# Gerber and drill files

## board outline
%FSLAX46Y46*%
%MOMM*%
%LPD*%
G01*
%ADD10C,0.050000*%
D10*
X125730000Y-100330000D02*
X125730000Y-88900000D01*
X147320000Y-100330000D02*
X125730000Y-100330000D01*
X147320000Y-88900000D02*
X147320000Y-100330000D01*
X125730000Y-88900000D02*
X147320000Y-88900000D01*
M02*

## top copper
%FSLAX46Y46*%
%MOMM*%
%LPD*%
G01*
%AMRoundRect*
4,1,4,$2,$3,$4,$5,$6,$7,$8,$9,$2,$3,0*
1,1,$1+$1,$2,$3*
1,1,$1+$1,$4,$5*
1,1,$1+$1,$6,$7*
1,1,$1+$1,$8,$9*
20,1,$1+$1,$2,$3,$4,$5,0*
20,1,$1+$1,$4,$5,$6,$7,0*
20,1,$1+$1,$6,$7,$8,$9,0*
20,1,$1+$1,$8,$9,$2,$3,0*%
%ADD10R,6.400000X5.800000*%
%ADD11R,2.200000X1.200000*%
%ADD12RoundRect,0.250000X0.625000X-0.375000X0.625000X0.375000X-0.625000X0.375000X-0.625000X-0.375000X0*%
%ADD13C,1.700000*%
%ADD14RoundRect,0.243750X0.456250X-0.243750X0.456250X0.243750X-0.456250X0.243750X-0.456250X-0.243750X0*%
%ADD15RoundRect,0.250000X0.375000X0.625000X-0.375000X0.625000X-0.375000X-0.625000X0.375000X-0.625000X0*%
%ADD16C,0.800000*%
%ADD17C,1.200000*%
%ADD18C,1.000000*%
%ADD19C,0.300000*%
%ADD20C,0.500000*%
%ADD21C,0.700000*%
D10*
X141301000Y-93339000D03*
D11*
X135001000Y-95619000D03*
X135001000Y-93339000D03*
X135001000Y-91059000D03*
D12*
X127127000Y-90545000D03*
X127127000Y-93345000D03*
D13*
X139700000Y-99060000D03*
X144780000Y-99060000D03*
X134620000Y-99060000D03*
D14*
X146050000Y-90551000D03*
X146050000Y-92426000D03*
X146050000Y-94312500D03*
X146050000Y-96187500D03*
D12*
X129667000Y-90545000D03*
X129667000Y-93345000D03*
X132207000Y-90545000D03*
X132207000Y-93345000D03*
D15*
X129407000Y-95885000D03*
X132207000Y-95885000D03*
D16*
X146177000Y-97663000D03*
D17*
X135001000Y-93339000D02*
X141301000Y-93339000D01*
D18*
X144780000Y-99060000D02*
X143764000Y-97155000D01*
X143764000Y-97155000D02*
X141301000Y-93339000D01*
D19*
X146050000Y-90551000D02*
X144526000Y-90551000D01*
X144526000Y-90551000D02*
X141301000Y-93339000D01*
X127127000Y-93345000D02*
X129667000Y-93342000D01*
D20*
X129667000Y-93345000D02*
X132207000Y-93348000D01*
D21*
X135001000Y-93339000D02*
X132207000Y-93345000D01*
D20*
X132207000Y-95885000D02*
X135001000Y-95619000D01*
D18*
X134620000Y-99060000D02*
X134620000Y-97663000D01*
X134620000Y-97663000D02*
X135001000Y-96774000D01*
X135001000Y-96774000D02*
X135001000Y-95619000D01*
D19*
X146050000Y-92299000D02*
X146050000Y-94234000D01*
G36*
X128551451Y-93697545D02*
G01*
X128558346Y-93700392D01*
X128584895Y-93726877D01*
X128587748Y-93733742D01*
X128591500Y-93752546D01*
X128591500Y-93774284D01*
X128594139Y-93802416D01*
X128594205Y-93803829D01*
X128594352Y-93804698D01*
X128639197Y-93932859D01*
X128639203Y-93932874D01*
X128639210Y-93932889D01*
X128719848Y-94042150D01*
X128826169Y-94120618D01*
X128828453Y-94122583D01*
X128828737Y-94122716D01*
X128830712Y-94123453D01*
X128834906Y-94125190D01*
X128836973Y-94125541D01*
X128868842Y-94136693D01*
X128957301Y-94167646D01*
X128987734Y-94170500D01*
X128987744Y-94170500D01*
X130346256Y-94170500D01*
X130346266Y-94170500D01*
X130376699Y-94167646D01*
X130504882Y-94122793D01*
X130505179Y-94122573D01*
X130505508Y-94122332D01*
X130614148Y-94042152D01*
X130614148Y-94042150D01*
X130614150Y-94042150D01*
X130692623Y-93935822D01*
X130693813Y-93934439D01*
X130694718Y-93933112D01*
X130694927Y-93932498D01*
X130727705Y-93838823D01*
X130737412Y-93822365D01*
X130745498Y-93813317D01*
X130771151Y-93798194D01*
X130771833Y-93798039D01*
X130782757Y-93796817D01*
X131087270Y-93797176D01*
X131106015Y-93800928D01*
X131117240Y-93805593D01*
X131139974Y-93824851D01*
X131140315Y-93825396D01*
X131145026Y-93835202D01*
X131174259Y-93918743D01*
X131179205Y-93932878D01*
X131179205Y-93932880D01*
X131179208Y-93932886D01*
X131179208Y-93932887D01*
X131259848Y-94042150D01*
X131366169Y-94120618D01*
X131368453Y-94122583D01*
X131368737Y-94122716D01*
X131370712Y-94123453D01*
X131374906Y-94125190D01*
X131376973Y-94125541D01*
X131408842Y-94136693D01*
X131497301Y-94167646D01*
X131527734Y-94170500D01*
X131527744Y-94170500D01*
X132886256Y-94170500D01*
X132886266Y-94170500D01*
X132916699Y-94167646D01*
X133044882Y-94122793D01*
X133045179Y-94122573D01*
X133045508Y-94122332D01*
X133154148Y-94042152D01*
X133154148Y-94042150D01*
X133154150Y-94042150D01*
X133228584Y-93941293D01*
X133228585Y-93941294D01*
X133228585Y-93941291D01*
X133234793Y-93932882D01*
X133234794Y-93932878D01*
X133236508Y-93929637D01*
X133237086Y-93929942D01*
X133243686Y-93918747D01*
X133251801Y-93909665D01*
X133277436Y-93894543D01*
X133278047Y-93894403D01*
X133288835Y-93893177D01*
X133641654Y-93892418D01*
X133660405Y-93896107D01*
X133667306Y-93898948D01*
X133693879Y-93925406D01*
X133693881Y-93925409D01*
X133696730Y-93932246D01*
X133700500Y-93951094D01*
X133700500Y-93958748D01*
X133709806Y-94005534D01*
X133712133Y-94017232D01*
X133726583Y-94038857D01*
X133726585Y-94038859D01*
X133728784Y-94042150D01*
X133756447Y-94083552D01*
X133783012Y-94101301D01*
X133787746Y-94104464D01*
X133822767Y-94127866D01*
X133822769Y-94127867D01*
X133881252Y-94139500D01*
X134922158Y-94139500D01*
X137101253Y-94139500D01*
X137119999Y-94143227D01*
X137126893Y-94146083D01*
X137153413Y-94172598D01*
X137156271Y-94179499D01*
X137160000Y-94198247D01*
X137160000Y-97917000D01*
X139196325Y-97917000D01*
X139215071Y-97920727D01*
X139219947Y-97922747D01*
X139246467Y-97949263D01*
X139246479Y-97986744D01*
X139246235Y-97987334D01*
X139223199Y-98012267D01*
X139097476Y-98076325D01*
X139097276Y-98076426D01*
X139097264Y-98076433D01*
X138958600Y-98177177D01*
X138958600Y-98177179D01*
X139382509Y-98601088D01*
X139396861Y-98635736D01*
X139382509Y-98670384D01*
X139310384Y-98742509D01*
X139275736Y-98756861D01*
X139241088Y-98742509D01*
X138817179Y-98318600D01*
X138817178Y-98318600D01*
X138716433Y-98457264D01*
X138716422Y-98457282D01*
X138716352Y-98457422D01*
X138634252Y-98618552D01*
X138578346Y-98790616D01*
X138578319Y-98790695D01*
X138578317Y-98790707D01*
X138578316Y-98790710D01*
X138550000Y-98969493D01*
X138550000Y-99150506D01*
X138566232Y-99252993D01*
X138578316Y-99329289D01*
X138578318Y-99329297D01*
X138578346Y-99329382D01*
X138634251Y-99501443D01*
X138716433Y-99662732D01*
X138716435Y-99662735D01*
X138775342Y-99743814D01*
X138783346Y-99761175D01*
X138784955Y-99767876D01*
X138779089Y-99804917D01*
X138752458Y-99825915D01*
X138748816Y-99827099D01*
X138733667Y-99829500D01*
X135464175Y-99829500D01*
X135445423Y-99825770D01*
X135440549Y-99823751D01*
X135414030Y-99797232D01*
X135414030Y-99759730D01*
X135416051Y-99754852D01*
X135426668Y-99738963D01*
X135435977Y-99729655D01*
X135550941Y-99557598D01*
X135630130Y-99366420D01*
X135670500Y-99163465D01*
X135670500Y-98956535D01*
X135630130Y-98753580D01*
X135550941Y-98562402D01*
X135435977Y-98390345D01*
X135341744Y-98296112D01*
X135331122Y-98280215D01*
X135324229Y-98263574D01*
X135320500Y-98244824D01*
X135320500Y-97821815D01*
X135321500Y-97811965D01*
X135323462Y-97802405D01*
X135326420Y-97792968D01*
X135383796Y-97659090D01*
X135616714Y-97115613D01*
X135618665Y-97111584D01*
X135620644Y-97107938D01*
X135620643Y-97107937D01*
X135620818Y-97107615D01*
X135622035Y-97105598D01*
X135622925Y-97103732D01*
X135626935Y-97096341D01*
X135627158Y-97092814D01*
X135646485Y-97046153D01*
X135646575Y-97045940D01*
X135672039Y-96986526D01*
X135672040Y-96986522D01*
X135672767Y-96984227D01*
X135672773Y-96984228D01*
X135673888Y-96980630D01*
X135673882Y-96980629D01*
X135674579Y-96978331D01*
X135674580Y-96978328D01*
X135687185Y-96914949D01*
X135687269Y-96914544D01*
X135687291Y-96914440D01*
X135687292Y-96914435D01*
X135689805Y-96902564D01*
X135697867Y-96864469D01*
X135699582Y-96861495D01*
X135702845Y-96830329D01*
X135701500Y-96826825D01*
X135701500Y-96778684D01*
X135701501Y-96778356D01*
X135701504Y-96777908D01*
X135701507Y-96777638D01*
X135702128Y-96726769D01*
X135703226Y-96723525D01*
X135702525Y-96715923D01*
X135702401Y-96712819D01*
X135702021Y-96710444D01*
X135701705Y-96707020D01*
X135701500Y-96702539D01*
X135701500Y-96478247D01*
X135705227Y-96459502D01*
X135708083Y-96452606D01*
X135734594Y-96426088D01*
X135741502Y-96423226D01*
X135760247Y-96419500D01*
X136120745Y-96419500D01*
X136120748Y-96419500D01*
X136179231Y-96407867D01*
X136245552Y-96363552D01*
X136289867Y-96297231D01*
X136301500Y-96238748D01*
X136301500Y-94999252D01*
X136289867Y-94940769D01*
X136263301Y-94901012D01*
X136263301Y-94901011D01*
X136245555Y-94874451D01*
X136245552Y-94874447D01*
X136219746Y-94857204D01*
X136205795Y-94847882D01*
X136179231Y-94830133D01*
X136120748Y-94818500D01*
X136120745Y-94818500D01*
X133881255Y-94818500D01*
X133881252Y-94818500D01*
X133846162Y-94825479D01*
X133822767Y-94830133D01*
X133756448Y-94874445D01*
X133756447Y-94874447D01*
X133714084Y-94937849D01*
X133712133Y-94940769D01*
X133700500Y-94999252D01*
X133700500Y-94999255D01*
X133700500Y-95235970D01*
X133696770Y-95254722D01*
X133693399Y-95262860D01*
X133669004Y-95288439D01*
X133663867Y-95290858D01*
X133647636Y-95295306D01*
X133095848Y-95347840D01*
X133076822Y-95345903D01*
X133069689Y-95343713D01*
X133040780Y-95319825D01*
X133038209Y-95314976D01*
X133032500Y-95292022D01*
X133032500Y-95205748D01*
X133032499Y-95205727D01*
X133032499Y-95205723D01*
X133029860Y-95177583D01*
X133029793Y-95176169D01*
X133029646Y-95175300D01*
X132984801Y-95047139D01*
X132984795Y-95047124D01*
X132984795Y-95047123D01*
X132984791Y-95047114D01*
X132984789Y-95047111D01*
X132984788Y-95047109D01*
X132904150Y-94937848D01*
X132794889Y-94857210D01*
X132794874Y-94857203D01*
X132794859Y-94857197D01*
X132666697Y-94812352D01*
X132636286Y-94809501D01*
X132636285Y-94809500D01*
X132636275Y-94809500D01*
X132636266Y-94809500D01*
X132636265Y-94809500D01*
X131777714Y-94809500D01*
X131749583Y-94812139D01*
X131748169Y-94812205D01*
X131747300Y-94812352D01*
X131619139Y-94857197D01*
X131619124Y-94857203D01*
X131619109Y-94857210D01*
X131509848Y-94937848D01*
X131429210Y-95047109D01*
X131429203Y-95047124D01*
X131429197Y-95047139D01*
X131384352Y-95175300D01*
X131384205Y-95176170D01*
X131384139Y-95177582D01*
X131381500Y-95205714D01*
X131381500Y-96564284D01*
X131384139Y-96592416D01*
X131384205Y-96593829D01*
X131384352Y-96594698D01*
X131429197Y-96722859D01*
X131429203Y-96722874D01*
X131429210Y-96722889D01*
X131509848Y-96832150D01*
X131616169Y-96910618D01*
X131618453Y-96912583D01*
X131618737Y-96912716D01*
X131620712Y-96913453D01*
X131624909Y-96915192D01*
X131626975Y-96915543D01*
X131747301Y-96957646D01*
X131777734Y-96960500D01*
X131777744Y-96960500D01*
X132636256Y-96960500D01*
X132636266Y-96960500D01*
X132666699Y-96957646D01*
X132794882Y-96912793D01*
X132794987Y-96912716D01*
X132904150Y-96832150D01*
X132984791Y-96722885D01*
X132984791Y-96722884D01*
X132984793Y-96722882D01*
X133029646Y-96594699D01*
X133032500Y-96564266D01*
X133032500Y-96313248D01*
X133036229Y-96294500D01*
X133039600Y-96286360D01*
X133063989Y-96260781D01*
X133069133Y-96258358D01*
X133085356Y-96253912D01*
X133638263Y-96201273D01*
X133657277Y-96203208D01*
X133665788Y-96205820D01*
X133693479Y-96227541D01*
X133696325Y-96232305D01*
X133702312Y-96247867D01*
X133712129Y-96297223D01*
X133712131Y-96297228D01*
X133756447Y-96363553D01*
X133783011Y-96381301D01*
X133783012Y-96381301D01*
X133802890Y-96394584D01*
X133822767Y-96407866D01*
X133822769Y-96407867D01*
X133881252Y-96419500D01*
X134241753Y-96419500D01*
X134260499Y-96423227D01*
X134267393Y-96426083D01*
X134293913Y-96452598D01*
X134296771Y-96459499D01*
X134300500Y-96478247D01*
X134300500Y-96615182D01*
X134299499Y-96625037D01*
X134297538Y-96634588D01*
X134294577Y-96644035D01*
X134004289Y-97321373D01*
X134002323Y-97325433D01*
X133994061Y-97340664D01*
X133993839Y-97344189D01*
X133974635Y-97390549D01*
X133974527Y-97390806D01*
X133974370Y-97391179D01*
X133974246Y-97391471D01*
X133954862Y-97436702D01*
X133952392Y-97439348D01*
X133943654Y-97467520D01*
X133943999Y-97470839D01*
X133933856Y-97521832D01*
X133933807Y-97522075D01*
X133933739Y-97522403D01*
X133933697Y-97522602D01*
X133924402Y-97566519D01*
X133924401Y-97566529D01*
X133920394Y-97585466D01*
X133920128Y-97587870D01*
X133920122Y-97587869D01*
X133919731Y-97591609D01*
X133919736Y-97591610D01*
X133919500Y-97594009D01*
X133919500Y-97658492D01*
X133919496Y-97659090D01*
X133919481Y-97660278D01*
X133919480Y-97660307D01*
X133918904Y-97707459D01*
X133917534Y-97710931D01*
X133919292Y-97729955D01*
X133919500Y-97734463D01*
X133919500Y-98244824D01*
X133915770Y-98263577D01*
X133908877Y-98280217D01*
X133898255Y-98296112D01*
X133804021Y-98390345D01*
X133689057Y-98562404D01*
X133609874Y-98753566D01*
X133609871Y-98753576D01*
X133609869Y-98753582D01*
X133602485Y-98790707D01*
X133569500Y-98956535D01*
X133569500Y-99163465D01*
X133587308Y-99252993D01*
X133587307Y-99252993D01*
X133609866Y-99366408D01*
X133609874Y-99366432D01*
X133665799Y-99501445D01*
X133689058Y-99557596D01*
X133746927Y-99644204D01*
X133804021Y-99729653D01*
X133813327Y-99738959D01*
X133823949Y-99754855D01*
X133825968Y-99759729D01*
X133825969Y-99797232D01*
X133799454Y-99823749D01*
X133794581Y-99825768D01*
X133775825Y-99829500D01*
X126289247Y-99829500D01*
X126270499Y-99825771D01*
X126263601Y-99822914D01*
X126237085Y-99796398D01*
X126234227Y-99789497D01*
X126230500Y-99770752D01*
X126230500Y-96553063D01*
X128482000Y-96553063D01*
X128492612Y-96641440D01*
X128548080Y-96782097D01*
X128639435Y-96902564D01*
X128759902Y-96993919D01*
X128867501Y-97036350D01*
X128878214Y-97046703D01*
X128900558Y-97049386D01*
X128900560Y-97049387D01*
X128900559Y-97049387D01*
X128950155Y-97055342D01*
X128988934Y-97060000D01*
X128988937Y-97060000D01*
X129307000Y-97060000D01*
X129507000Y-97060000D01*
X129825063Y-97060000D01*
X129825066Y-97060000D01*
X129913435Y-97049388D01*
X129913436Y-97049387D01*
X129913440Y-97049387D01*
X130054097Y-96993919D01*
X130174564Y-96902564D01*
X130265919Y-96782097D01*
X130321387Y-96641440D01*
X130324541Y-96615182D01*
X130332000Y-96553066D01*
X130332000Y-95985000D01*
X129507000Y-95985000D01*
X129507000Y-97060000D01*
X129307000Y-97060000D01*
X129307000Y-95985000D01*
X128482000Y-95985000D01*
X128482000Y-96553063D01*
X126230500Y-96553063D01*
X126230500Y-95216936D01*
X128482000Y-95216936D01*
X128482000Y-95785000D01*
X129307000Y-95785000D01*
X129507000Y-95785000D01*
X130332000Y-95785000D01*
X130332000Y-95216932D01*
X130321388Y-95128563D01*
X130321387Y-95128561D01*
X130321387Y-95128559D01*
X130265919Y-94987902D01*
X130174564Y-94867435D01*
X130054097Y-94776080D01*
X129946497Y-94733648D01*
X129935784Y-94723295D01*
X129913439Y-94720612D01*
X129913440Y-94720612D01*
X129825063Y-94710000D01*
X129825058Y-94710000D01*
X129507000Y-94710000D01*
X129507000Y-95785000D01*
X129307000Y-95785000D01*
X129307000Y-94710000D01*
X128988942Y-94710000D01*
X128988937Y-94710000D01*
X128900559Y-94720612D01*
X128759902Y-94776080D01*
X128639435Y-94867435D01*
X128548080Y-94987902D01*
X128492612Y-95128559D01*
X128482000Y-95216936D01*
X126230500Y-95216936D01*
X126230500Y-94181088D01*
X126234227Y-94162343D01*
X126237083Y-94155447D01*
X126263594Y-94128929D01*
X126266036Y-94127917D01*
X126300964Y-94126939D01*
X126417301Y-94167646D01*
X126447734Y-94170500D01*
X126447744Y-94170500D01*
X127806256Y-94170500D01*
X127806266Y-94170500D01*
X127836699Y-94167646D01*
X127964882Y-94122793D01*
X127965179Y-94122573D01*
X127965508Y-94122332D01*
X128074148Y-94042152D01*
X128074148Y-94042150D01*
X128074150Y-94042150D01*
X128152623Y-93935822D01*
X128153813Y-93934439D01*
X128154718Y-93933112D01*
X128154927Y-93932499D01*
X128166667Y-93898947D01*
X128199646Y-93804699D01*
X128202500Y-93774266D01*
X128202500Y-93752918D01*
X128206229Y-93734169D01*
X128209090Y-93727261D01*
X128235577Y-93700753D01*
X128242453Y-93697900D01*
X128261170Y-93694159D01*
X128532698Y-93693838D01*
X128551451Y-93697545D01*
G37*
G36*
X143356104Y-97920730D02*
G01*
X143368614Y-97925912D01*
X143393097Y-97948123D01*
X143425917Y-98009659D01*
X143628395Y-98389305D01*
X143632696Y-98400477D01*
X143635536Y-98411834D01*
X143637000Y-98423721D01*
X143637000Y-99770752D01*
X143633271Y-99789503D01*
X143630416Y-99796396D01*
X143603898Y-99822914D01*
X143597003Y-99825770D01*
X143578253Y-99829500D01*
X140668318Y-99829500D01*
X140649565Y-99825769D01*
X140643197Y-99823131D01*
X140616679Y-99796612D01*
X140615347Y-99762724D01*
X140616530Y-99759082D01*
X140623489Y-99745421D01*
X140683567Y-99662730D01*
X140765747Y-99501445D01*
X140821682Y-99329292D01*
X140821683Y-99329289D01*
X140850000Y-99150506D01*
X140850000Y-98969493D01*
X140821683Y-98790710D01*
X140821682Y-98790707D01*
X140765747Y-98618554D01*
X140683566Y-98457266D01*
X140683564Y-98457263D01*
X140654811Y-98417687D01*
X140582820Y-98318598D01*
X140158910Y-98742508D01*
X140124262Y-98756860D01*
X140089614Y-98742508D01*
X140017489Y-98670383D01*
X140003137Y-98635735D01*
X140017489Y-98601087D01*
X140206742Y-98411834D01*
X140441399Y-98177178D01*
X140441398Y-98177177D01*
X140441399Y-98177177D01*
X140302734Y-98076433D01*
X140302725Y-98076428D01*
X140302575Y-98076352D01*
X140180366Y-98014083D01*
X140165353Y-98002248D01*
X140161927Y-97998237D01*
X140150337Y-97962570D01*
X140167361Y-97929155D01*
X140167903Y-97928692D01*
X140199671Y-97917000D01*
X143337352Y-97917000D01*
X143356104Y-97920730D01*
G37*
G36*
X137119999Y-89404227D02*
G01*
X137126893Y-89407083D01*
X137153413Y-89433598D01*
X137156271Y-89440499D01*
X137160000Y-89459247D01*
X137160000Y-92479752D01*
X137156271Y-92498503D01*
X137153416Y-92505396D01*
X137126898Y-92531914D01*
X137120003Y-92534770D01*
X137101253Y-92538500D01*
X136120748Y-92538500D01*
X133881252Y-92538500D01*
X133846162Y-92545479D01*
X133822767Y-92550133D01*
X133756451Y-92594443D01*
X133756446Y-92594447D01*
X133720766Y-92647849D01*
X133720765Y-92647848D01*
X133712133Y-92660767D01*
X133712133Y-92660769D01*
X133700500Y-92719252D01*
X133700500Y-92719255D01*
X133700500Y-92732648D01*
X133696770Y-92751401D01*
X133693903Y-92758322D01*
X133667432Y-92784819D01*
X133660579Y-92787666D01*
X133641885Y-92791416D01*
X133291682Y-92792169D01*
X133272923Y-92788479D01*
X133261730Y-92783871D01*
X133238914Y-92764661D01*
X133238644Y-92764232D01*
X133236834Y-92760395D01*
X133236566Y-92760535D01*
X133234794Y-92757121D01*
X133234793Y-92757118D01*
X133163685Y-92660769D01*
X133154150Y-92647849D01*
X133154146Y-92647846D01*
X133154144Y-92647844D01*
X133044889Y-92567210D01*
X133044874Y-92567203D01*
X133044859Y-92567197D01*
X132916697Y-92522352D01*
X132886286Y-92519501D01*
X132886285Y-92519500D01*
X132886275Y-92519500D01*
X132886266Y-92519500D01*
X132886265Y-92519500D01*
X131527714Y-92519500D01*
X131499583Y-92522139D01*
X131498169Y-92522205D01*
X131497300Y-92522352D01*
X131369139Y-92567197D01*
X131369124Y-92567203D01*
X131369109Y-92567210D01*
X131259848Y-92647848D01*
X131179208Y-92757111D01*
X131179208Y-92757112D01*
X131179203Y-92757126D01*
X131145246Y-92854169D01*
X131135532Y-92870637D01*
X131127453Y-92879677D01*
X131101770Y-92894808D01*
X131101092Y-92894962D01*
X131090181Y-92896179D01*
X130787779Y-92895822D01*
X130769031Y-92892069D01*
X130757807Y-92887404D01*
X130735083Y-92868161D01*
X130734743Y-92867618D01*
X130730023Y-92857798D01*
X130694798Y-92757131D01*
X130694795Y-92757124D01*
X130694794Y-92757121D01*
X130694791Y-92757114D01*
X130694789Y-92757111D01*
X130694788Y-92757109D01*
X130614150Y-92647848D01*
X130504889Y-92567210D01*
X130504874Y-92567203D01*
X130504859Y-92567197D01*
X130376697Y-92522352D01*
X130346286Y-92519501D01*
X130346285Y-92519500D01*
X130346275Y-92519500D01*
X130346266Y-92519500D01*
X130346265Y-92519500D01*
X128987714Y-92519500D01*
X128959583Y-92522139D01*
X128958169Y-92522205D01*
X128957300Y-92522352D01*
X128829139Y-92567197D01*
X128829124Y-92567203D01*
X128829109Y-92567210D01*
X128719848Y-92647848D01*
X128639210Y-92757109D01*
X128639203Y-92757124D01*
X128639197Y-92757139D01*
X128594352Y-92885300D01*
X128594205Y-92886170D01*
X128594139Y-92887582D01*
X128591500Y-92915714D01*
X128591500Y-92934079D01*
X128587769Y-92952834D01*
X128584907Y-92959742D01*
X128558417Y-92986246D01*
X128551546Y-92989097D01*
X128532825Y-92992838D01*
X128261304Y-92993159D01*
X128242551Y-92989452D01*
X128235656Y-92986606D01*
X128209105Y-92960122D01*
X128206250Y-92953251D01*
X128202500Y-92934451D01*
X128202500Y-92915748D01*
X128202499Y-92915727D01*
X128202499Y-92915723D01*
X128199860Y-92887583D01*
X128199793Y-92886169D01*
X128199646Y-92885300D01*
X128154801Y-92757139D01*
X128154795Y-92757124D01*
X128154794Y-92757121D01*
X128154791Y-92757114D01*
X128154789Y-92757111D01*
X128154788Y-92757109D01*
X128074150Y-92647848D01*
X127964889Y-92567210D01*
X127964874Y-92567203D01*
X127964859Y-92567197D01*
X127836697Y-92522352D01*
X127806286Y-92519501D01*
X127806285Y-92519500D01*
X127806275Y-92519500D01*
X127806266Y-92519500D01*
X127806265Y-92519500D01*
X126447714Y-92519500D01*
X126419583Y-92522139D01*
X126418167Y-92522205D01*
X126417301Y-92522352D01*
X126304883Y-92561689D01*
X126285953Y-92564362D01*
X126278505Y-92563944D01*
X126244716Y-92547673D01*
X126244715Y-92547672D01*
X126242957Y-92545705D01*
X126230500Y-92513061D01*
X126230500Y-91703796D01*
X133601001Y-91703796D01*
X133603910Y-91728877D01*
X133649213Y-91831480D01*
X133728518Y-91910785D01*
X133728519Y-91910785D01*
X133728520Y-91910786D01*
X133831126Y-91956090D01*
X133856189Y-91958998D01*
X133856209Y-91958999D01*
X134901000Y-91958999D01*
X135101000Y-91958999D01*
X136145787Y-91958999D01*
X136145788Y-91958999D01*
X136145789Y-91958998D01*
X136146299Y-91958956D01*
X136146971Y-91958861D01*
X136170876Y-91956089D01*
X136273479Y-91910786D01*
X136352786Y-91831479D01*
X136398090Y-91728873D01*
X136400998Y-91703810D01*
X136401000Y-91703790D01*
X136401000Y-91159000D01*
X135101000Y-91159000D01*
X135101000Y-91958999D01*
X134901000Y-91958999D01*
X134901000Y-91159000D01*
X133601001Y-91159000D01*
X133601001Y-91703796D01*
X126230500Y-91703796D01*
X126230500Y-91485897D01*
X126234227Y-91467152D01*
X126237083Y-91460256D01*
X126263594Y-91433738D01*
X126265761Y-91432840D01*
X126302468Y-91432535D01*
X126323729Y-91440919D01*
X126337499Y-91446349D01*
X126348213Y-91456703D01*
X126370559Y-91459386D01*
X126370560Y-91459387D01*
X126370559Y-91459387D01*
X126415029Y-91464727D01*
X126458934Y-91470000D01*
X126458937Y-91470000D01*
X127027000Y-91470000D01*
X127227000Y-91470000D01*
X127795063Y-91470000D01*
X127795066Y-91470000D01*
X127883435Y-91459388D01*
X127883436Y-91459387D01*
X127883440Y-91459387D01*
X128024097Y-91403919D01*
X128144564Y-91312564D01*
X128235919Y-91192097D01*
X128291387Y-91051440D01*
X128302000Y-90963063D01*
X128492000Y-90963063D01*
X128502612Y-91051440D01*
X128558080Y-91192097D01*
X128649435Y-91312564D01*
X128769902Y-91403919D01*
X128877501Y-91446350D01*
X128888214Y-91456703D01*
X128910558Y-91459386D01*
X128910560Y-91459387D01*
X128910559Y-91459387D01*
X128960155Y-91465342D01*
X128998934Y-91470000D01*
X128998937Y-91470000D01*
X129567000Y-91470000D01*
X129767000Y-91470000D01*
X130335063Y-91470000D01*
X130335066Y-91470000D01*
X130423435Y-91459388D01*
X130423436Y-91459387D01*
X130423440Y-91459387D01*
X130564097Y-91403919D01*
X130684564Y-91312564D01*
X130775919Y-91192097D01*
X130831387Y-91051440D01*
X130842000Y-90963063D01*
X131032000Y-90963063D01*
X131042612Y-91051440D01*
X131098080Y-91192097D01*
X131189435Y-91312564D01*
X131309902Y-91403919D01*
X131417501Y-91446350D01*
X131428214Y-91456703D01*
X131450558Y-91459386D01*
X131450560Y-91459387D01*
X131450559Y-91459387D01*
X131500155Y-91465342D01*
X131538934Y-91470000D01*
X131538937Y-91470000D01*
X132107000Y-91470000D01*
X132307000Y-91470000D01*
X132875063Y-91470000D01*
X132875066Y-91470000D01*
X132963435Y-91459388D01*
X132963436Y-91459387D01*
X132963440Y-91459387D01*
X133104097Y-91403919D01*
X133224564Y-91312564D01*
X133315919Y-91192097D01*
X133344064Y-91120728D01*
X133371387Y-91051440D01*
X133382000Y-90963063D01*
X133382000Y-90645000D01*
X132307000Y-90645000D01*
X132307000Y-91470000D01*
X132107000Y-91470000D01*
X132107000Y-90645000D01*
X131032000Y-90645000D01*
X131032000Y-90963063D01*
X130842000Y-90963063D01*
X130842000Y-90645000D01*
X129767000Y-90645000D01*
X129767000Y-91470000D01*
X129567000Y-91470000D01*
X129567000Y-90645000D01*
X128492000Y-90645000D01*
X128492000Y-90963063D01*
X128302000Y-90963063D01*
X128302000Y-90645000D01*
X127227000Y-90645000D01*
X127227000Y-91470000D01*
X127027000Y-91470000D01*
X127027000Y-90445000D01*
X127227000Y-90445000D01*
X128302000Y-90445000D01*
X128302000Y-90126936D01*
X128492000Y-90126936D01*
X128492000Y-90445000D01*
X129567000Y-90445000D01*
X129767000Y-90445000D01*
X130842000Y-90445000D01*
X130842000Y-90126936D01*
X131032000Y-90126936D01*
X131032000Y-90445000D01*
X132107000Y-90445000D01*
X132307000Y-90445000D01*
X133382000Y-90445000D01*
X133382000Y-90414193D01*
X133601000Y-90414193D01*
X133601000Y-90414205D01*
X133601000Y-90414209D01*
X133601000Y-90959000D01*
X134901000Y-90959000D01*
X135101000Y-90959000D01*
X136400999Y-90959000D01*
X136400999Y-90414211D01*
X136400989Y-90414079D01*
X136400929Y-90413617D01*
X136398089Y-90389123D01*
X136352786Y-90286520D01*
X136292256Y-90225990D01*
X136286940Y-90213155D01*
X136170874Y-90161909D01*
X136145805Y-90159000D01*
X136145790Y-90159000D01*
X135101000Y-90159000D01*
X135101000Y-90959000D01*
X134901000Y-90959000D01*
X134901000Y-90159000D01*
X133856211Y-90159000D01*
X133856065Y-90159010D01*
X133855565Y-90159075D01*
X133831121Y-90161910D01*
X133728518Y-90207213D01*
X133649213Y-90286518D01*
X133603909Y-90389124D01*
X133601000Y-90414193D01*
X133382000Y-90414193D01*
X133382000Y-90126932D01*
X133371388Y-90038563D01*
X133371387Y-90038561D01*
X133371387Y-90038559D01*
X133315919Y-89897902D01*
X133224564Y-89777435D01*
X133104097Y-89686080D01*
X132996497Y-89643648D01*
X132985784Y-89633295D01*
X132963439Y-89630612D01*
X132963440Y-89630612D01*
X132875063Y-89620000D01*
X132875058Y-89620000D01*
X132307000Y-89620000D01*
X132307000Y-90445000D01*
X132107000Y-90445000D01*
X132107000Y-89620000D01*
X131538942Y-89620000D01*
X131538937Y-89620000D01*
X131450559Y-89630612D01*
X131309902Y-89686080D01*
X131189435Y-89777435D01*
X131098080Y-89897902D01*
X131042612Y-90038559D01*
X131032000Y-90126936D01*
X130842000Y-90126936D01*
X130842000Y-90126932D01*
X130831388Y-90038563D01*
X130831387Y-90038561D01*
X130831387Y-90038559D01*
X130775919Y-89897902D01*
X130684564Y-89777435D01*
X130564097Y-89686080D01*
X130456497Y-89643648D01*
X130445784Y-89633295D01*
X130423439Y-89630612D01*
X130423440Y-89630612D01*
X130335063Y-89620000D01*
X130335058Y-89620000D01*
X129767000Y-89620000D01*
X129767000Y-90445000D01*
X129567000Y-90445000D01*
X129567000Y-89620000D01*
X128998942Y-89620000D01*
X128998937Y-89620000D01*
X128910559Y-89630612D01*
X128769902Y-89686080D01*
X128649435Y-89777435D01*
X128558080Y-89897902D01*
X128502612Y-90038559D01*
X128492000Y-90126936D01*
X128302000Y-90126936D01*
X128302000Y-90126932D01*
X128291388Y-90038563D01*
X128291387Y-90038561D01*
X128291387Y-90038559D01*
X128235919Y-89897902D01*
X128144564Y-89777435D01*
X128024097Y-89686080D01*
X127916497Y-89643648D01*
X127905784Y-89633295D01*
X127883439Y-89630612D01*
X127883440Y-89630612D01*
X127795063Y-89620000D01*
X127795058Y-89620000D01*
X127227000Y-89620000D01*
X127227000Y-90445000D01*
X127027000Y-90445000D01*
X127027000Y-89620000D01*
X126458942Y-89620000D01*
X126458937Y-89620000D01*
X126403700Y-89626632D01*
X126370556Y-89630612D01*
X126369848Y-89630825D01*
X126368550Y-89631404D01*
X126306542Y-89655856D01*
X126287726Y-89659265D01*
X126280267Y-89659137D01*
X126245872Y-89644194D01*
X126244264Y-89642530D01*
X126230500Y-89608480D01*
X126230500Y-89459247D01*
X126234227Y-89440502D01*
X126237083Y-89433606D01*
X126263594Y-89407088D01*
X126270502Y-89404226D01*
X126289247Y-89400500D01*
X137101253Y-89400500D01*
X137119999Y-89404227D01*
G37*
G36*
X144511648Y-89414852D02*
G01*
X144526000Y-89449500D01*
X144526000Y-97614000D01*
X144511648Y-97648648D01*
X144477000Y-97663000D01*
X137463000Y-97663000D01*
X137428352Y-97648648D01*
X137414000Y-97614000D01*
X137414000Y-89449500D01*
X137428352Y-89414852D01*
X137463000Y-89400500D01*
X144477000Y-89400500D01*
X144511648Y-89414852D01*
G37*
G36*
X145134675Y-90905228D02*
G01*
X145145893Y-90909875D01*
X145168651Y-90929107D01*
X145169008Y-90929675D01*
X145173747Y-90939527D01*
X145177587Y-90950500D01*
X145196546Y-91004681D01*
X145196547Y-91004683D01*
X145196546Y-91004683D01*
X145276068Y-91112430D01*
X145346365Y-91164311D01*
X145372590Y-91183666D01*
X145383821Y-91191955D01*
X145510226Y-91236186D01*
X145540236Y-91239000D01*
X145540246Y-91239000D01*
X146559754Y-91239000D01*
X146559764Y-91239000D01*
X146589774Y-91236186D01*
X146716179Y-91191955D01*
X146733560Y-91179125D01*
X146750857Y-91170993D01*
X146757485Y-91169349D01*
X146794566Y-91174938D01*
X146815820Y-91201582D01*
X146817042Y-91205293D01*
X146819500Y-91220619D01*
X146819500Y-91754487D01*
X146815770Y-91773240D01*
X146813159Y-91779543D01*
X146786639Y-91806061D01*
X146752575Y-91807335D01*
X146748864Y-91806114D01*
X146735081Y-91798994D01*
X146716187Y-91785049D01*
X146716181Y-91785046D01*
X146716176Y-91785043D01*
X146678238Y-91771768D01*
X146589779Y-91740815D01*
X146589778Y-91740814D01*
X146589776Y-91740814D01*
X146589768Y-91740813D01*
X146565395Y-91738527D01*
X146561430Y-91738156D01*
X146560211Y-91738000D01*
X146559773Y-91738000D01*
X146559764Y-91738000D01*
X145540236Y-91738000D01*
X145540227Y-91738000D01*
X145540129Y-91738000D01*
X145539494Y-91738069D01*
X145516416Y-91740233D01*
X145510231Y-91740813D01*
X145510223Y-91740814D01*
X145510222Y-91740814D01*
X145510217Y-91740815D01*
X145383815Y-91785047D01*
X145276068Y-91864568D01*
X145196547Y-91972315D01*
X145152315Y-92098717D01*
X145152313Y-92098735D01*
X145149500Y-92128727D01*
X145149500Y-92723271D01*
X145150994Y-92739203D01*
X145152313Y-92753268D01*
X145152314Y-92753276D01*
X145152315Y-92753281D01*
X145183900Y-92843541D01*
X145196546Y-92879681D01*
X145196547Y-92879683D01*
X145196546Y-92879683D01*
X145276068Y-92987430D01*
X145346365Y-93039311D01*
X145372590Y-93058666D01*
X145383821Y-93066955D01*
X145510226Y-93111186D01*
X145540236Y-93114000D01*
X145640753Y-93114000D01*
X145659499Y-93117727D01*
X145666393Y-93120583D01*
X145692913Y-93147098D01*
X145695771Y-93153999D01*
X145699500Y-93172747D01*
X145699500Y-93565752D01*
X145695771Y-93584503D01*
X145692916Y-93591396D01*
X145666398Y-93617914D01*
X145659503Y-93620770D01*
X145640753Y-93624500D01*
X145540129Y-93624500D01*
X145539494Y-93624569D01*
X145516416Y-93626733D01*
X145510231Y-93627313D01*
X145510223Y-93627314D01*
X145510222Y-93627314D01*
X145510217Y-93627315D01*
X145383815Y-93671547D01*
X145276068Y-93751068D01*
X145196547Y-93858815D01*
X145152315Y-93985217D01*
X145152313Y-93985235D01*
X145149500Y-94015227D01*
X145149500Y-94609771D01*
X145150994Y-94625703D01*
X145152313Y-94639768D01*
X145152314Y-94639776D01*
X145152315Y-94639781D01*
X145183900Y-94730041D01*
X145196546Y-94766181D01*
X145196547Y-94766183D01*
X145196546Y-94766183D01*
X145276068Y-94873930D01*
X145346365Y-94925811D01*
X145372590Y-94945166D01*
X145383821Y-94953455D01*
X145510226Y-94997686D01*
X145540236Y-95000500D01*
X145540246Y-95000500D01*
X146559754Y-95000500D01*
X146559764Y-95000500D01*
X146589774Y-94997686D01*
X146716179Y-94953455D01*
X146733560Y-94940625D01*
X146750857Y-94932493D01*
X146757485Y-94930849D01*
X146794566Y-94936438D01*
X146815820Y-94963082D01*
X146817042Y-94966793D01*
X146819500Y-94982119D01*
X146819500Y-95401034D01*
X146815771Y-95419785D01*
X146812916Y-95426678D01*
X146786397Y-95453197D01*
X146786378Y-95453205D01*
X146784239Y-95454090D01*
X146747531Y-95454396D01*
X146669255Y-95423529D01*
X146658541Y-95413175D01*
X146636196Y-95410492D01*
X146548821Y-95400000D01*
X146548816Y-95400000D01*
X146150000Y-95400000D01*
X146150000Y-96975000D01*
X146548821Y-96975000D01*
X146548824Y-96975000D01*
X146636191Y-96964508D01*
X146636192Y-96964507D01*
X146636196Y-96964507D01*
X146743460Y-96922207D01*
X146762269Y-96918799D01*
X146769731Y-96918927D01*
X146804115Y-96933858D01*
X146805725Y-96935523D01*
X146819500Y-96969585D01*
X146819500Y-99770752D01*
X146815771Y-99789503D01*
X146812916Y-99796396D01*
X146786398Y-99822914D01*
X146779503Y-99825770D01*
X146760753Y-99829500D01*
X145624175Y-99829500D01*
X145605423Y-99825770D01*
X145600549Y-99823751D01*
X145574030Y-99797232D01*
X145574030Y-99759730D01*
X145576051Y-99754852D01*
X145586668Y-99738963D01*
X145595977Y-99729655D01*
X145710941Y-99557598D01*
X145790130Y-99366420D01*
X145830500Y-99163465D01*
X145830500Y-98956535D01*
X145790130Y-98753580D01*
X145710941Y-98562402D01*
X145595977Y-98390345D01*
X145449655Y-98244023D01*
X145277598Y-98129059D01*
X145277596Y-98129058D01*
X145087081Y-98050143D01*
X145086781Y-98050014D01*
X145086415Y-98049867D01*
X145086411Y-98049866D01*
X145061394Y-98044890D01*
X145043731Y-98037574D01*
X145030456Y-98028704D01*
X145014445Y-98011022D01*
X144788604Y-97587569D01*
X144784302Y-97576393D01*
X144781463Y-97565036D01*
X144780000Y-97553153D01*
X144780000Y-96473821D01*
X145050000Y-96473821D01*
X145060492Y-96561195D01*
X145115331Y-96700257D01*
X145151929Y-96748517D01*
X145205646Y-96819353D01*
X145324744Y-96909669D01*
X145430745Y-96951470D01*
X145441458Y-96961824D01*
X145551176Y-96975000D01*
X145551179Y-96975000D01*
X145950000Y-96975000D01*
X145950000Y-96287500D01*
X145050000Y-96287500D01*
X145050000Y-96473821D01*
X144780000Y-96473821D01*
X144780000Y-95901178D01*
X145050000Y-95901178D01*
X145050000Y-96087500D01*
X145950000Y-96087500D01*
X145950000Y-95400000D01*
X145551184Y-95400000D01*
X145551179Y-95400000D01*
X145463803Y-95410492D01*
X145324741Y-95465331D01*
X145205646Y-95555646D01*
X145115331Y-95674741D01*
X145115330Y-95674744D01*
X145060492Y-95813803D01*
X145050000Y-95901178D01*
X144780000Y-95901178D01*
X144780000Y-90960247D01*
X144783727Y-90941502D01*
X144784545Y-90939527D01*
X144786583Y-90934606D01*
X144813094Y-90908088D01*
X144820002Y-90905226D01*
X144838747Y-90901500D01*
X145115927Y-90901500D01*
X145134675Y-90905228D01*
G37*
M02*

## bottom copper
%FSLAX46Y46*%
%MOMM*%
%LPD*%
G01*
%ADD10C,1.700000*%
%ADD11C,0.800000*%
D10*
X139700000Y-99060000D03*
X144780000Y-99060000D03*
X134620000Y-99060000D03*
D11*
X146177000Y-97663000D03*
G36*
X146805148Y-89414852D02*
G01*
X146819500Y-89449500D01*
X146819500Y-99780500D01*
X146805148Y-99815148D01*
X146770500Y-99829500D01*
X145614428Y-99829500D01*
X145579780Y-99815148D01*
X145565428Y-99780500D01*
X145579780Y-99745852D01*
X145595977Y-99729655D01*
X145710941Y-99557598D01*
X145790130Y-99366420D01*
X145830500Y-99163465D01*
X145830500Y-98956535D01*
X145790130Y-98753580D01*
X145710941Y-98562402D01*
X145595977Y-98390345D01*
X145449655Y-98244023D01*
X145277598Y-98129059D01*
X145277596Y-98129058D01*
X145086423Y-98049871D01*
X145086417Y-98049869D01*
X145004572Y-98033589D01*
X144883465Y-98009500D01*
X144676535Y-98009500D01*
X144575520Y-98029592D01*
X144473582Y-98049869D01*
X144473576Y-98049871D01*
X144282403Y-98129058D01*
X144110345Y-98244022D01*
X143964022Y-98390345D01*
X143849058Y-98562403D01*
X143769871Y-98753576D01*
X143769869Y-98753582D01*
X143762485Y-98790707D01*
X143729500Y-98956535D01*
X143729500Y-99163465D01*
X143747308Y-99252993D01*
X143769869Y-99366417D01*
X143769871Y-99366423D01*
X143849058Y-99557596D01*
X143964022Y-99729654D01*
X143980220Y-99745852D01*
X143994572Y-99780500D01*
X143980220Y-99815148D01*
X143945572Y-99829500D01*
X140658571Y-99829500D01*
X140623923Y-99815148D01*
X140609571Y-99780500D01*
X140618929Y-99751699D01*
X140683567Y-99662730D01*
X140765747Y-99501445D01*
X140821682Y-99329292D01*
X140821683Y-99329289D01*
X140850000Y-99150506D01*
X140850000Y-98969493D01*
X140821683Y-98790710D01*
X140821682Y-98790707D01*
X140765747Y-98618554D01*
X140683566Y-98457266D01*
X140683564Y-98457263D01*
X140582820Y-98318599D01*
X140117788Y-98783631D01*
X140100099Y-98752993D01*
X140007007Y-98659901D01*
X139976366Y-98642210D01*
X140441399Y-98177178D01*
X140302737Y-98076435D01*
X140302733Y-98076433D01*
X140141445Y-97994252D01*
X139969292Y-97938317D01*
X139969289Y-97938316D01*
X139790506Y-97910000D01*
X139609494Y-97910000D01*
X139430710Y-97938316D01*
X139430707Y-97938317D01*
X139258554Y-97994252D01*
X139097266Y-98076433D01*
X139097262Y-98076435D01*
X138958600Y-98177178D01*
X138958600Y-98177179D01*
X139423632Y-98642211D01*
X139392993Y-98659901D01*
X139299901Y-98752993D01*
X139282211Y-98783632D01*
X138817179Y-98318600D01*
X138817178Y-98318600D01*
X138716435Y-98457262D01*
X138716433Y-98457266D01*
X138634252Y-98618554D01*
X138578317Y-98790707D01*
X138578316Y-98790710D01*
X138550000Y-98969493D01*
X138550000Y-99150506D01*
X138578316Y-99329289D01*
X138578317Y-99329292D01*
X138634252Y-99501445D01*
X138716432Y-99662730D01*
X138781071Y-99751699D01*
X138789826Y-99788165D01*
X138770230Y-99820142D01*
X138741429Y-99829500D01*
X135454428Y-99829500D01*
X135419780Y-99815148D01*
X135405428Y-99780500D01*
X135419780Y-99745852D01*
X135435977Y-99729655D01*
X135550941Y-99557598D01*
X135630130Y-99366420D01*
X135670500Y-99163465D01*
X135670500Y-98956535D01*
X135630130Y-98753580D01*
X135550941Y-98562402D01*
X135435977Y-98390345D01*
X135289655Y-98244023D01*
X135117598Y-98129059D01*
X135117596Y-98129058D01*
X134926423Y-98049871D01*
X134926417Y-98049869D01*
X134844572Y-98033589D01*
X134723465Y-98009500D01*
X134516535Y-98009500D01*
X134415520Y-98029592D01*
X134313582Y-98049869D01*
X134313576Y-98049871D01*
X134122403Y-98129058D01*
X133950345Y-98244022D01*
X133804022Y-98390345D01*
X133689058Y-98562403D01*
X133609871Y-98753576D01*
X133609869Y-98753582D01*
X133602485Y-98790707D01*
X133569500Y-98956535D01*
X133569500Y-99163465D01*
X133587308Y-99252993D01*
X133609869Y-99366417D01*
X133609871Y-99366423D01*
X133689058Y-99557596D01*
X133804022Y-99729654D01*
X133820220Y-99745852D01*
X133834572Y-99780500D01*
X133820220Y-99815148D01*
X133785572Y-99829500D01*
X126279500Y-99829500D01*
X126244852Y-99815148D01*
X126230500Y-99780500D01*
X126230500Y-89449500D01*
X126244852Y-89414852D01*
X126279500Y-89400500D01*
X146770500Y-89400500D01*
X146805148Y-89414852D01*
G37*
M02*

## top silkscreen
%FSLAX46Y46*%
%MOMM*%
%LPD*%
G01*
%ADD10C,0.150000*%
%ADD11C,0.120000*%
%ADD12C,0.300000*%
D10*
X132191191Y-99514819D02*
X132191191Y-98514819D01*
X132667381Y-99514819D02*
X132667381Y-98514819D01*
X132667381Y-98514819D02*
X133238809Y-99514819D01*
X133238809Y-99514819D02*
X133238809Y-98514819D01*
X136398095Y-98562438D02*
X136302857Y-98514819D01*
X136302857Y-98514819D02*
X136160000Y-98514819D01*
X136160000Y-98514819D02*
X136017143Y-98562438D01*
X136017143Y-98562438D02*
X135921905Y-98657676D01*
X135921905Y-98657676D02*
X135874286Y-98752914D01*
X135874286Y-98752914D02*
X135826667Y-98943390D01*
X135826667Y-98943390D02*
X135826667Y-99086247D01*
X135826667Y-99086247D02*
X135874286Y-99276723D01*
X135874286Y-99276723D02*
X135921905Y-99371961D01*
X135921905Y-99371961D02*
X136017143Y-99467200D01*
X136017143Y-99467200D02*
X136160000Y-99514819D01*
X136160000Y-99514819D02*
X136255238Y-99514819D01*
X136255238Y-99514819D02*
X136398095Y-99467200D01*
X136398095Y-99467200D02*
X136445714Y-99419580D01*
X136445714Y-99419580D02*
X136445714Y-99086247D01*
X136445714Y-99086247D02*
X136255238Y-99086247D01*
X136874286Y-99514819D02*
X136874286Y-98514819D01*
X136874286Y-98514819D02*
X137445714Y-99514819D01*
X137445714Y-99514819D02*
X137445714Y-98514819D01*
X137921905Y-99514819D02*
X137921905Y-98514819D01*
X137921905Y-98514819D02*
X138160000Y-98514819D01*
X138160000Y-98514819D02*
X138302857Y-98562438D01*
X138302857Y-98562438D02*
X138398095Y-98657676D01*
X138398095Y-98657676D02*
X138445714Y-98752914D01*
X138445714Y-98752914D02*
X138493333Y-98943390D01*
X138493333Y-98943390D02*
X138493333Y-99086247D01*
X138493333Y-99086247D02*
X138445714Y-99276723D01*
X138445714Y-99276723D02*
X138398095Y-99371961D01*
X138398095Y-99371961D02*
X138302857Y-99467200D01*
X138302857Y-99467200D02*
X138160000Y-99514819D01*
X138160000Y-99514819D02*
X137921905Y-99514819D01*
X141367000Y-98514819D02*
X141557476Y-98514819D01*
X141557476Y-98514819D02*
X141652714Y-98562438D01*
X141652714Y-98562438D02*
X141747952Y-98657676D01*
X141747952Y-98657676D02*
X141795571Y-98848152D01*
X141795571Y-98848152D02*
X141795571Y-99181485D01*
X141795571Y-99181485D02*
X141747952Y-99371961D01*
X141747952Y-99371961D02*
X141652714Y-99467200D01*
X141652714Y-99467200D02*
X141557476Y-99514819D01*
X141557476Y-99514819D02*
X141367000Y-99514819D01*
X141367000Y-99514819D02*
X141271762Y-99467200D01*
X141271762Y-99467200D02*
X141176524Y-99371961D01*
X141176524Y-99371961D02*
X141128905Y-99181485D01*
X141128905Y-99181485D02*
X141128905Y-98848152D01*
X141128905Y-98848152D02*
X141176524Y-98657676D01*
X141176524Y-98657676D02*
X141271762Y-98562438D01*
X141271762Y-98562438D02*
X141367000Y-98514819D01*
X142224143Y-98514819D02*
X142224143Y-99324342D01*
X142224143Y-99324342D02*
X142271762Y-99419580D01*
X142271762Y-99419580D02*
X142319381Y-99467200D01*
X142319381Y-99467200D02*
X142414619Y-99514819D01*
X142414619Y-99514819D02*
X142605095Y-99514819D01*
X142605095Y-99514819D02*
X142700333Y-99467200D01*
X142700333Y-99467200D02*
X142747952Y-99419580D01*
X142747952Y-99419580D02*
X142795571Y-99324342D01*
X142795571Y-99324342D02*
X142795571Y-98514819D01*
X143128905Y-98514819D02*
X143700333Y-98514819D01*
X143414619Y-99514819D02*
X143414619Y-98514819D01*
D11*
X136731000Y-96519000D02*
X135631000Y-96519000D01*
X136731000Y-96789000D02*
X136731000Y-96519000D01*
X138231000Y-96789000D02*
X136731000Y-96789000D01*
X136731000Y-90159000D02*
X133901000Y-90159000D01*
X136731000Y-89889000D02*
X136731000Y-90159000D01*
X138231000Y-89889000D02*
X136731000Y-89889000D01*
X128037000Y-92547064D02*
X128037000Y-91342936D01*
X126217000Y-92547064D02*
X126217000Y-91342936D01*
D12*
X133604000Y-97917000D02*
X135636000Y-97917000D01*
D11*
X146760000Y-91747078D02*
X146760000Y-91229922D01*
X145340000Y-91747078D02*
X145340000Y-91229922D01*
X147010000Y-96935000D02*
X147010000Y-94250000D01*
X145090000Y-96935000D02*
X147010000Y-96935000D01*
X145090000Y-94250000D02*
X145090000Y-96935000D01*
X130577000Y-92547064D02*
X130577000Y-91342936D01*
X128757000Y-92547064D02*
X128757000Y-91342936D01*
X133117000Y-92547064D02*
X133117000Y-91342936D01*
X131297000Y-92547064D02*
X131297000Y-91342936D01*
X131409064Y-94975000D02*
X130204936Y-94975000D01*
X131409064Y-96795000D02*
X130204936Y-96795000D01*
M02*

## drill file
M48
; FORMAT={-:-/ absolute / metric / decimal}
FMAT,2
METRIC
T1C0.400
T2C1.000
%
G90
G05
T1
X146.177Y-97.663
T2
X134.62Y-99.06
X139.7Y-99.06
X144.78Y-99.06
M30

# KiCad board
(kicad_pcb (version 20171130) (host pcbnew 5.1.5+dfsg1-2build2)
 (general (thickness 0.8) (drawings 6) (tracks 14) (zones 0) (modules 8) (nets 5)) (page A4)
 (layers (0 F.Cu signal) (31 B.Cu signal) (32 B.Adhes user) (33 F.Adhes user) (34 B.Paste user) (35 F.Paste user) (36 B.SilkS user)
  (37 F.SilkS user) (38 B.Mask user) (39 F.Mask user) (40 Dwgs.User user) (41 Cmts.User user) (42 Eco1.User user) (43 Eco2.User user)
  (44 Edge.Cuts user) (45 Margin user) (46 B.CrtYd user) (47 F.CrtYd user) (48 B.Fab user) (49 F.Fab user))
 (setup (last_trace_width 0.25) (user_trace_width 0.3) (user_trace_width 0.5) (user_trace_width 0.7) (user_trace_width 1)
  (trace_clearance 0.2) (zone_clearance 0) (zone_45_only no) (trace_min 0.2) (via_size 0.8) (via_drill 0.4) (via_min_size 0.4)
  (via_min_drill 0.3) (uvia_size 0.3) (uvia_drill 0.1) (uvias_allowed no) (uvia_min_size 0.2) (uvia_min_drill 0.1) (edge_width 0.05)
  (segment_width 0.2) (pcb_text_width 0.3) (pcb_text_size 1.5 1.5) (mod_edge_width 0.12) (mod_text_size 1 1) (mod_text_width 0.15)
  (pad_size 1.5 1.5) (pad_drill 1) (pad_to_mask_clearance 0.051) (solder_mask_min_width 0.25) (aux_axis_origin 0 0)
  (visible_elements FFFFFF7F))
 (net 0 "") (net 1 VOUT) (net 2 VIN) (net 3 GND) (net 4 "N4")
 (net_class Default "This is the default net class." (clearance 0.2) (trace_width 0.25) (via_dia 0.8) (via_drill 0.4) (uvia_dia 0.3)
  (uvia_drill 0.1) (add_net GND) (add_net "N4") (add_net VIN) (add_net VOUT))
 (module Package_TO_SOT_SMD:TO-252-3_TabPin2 (layer F.Cu) (at 139.201 93.339)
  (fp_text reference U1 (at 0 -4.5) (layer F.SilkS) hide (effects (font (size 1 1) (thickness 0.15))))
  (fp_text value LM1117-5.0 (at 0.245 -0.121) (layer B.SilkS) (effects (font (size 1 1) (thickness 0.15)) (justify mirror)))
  (fp_line (start -2.47 3.18) (end -3.57 3.18) (layer F.SilkS) (width 0.12))
  (fp_line (start -2.47 3.45) (end -2.47 3.18) (layer F.SilkS) (width 0.12))
  (fp_line (start -0.97 3.45) (end -2.47 3.45) (layer F.SilkS) (width 0.12))
  (fp_line (start -2.47 -3.18) (end -5.3 -3.18) (layer F.SilkS) (width 0.12))
  (fp_line (start -2.47 -3.45) (end -2.47 -3.18) (layer F.SilkS) (width 0.12))
  (fp_line (start -0.97 -3.45) (end -2.47 -3.45) (layer F.SilkS) (width 0.12))
  (pad "" smd rect (at 0.425 1.525) (size 3.05 2.75) (layers F.Paste))
  (pad "" smd rect (at 3.775 -1.525) (size 3.05 2.75) (layers F.Paste))
  (pad "" smd rect (at 0.425 -1.525) (size 3.05 2.75) (layers F.Paste))
  (pad "" smd rect (at 3.775 1.525) (size 3.05 2.75) (layers F.Paste))
  (pad 2 smd rect (at 2.1 0) (size 6.4 5.8) (layers F.Cu F.Mask) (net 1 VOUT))
  (pad 3 smd rect (at -4.2 2.28) (size 2.2 1.2) (layers F.Cu F.Paste F.Mask) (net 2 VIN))
  (pad 2 smd rect (at -4.2 0) (size 2.2 1.2) (layers F.Cu F.Paste F.Mask) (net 1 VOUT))
  (pad 1 smd rect (at -4.2 -2.28) (size 2.2 1.2) (layers F.Cu F.Paste F.Mask) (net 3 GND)))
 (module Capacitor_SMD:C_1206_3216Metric (layer F.Cu) (at 127.127 91.945 90)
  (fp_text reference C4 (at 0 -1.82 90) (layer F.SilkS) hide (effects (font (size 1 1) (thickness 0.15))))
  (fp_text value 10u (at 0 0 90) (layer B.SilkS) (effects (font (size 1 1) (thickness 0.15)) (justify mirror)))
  (fp_line (start -0.602064 0.91) (end 0.602064 0.91) (layer F.SilkS) (width 0.12))
  (fp_line (start -0.602064 -0.91) (end 0.602064 -0.91) (layer F.SilkS) (width 0.12))
  (pad 2 smd roundrect (at 1.4 0 90) (size 1.25 1.75) (layers F.Cu F.Paste F.Mask) (roundrect_rratio 0.2) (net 3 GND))
  (pad 1 smd roundrect (at -1.4 0 90) (size 1.25 1.75) (layers F.Cu F.Paste F.Mask) (roundrect_rratio 0.2) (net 1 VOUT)))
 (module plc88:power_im (layer F.Cu) (at 128.27 88.9)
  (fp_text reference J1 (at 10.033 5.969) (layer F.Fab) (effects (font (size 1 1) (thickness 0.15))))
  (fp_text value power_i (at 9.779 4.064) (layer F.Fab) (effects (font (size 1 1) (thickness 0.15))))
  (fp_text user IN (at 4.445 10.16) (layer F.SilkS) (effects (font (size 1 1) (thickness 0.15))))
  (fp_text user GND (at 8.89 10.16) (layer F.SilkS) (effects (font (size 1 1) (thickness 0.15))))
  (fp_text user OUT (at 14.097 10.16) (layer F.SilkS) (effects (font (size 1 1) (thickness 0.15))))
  (fp_line (start 5.334 9.017) (end 7.366 9.017) (layer F.SilkS) (width 0.3))
  (pad 3 thru_hole circle (at 11.43 10.16) (size 1.7 1.7) (drill 1) (layers *.Cu *.Mask) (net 3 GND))
  (pad 2 thru_hole circle (at 16.51 10.16) (size 1.7 1.7) (drill 1) (layers *.Cu *.Mask) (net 1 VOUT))
  (pad 1 thru_hole circle (at 6.35 10.16) (size 1.7 1.7) (drill 1) (layers *.Cu *.Mask) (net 2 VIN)))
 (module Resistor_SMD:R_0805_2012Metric (layer F.Cu) (at 146.05 91.4885 90)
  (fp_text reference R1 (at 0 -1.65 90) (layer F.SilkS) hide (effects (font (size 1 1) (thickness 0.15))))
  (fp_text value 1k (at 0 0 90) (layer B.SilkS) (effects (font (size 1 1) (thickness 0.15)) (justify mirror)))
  (fp_line (start -0.258578 0.71) (end 0.258578 0.71) (layer F.SilkS) (width 0.12))
  (fp_line (start -0.258578 -0.71) (end 0.258578 -0.71) (layer F.SilkS) (width 0.12))
  (pad 2 smd roundrect (at 0.9375 0 90) (size 0.975 1.4) (layers F.Cu F.Paste F.Mask) (roundrect_rratio 0.25) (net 1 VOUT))
  (pad 1 smd roundrect (at -0.9375 0 90) (size 0.975 1.4) (layers F.Cu F.Paste F.Mask) (roundrect_rratio 0.25) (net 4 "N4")))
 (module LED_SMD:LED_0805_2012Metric (layer F.Cu) (at 146.05 95.25 90)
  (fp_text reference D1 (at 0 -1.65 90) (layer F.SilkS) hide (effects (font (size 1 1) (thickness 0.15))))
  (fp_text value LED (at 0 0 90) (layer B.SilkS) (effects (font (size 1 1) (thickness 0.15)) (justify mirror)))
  (fp_line (start -1.685 0.96) (end 1 0.96) (layer F.SilkS) (width 0.12))
  (fp_line (start -1.685 -0.96) (end -1.685 0.96) (layer F.SilkS) (width 0.12))
  (fp_line (start 1 -0.96) (end -1.685 -0.96) (layer F.SilkS) (width 0.12))
  (pad 2 smd roundrect (at 0.9375 0 90) (size 0.975 1.4) (layers F.Cu F.Paste F.Mask) (roundrect_rratio 0.25) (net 4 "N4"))
  (pad 1 smd roundrect (at -0.9375 0 90) (size 0.975 1.4) (layers F.Cu F.Paste F.Mask) (roundrect_rratio 0.25) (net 3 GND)))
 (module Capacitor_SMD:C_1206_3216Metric (layer F.Cu) (at 129.667 91.945 90)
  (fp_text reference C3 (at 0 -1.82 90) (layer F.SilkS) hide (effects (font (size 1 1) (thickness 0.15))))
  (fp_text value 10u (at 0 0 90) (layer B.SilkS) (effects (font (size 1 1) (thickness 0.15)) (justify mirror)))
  (fp_line (start -0.602064 0.91) (end 0.602064 0.91) (layer F.SilkS) (width 0.12))
  (fp_line (start -0.602064 -0.91) (end 0.602064 -0.91) (layer F.SilkS) (width 0.12))
  (pad 2 smd roundrect (at 1.4 0 90) (size 1.25 1.75) (layers F.Cu F.Paste F.Mask) (roundrect_rratio 0.2) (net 3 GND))
  (pad 1 smd roundrect (at -1.4 0 90) (size 1.25 1.75) (layers F.Cu F.Paste F.Mask) (roundrect_rratio 0.2) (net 1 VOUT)))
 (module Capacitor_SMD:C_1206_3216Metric (layer F.Cu) (at 132.207 91.945 90)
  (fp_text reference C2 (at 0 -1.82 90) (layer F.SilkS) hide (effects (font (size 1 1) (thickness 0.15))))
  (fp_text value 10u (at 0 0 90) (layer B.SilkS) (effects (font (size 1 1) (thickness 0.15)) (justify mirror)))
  (fp_line (start -0.602064 0.91) (end 0.602064 0.91) (layer F.SilkS) (width 0.12))
  (fp_line (start -0.602064 -0.91) (end 0.602064 -0.91) (layer F.SilkS) (width 0.12))
  (pad 2 smd roundrect (at 1.4 0 90) (size 1.25 1.75) (layers F.Cu F.Paste F.Mask) (roundrect_rratio 0.2) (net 3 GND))
  (pad 1 smd roundrect (at -1.4 0 90) (size 1.25 1.75) (layers F.Cu F.Paste F.Mask) (roundrect_rratio 0.2) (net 1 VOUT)))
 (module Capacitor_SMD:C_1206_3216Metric (layer F.Cu) (at 130.807 95.885 180)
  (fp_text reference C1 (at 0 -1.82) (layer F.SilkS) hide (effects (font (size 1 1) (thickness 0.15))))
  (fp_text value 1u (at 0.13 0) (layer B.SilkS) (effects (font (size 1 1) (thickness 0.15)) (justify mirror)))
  (fp_line (start -0.602064 0.91) (end 0.602064 0.91) (layer F.SilkS) (width 0.12))
  (fp_line (start -0.602064 -0.91) (end 0.602064 -0.91) (layer F.SilkS) (width 0.12))
  (pad 2 smd roundrect (at 1.4 0 180) (size 1.25 1.75) (layers F.Cu F.Paste F.Mask) (roundrect_rratio 0.2) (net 3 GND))
  (pad 1 smd roundrect (at -1.4 0 180) (size 1.25 1.75) (layers F.Cu F.Paste F.Mask) (roundrect_rratio 0.2) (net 2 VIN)))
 (gr_line (start 125.73 100.33) (end 125.73 88.9) (layer Edge.Cuts) (width 0.05))
 (gr_line (start 147.32 100.33) (end 125.73 100.33) (layer Edge.Cuts) (width 0.05))
 (gr_line (start 147.32 88.9) (end 147.32 100.33) (layer Edge.Cuts) (width 0.05))
 (gr_line (start 125.73 88.9) (end 147.32 88.9) (layer Edge.Cuts) (width 0.05))
 (segment (start 135.001 93.339) (end 141.301 93.339) (width 1.2) (layer F.Cu) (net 1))
 (segment (start 144.78 99.06) (end 143.764 97.155) (width 1) (layer F.Cu) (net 1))
 (segment (start 143.764 97.155) (end 141.301 93.339) (width 1) (layer F.Cu) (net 1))
 (segment (start 146.05 90.551) (end 144.526 90.551) (width 0.3) (layer F.Cu) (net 1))
 (segment (start 144.526 90.551) (end 141.301 93.339) (width 0.3) (layer F.Cu) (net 1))
 (segment (start 127.127 93.345) (end 129.667 93.342) (width 0.3) (layer F.Cu) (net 1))
 (segment (start 129.667 93.345) (end 132.207 93.348) (width 0.5) (layer F.Cu) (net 1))
 (segment (start 135.001 93.339) (end 132.207 93.345) (width 0.7) (layer F.Cu) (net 1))
 (segment (start 132.207 95.885) (end 135.001 95.619) (width 0.5) (layer F.Cu) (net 2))
 (segment (start 134.62 99.06) (end 134.62 97.663) (width 1) (layer F.Cu) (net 2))
 (segment (start 134.62 97.663) (end 135.001 96.774) (width 1) (layer F.Cu) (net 2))
 (segment (start 135.001 96.774) (end 135.001 95.619) (width 1) (layer F.Cu) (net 2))
 (via (at 146.177 97.663) (size 0.8) (drill 0.4) (layers F.Cu B.Cu) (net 3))
 (segment (start 146.05 92.299) (end 146.05 94.234) (width 0.3) (layer F.Cu) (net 4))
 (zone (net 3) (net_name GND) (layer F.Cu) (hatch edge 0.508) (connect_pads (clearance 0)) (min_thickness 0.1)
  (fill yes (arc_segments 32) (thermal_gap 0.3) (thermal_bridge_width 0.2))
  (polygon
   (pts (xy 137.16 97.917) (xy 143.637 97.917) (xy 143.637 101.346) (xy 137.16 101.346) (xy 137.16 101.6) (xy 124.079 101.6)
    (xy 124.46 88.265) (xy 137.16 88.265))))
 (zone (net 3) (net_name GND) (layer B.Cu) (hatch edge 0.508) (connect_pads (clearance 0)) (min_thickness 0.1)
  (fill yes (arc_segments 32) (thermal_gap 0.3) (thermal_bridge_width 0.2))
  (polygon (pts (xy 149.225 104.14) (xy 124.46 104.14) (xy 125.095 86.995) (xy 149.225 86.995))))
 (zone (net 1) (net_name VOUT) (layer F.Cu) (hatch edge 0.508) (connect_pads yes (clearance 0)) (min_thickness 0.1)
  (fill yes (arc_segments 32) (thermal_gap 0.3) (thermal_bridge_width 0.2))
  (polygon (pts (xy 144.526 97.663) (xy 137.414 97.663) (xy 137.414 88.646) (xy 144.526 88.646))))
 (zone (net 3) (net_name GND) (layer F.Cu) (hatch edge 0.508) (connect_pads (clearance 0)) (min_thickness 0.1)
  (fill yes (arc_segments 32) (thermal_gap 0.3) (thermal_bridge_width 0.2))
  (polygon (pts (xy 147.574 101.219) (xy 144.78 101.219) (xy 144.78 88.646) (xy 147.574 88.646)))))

